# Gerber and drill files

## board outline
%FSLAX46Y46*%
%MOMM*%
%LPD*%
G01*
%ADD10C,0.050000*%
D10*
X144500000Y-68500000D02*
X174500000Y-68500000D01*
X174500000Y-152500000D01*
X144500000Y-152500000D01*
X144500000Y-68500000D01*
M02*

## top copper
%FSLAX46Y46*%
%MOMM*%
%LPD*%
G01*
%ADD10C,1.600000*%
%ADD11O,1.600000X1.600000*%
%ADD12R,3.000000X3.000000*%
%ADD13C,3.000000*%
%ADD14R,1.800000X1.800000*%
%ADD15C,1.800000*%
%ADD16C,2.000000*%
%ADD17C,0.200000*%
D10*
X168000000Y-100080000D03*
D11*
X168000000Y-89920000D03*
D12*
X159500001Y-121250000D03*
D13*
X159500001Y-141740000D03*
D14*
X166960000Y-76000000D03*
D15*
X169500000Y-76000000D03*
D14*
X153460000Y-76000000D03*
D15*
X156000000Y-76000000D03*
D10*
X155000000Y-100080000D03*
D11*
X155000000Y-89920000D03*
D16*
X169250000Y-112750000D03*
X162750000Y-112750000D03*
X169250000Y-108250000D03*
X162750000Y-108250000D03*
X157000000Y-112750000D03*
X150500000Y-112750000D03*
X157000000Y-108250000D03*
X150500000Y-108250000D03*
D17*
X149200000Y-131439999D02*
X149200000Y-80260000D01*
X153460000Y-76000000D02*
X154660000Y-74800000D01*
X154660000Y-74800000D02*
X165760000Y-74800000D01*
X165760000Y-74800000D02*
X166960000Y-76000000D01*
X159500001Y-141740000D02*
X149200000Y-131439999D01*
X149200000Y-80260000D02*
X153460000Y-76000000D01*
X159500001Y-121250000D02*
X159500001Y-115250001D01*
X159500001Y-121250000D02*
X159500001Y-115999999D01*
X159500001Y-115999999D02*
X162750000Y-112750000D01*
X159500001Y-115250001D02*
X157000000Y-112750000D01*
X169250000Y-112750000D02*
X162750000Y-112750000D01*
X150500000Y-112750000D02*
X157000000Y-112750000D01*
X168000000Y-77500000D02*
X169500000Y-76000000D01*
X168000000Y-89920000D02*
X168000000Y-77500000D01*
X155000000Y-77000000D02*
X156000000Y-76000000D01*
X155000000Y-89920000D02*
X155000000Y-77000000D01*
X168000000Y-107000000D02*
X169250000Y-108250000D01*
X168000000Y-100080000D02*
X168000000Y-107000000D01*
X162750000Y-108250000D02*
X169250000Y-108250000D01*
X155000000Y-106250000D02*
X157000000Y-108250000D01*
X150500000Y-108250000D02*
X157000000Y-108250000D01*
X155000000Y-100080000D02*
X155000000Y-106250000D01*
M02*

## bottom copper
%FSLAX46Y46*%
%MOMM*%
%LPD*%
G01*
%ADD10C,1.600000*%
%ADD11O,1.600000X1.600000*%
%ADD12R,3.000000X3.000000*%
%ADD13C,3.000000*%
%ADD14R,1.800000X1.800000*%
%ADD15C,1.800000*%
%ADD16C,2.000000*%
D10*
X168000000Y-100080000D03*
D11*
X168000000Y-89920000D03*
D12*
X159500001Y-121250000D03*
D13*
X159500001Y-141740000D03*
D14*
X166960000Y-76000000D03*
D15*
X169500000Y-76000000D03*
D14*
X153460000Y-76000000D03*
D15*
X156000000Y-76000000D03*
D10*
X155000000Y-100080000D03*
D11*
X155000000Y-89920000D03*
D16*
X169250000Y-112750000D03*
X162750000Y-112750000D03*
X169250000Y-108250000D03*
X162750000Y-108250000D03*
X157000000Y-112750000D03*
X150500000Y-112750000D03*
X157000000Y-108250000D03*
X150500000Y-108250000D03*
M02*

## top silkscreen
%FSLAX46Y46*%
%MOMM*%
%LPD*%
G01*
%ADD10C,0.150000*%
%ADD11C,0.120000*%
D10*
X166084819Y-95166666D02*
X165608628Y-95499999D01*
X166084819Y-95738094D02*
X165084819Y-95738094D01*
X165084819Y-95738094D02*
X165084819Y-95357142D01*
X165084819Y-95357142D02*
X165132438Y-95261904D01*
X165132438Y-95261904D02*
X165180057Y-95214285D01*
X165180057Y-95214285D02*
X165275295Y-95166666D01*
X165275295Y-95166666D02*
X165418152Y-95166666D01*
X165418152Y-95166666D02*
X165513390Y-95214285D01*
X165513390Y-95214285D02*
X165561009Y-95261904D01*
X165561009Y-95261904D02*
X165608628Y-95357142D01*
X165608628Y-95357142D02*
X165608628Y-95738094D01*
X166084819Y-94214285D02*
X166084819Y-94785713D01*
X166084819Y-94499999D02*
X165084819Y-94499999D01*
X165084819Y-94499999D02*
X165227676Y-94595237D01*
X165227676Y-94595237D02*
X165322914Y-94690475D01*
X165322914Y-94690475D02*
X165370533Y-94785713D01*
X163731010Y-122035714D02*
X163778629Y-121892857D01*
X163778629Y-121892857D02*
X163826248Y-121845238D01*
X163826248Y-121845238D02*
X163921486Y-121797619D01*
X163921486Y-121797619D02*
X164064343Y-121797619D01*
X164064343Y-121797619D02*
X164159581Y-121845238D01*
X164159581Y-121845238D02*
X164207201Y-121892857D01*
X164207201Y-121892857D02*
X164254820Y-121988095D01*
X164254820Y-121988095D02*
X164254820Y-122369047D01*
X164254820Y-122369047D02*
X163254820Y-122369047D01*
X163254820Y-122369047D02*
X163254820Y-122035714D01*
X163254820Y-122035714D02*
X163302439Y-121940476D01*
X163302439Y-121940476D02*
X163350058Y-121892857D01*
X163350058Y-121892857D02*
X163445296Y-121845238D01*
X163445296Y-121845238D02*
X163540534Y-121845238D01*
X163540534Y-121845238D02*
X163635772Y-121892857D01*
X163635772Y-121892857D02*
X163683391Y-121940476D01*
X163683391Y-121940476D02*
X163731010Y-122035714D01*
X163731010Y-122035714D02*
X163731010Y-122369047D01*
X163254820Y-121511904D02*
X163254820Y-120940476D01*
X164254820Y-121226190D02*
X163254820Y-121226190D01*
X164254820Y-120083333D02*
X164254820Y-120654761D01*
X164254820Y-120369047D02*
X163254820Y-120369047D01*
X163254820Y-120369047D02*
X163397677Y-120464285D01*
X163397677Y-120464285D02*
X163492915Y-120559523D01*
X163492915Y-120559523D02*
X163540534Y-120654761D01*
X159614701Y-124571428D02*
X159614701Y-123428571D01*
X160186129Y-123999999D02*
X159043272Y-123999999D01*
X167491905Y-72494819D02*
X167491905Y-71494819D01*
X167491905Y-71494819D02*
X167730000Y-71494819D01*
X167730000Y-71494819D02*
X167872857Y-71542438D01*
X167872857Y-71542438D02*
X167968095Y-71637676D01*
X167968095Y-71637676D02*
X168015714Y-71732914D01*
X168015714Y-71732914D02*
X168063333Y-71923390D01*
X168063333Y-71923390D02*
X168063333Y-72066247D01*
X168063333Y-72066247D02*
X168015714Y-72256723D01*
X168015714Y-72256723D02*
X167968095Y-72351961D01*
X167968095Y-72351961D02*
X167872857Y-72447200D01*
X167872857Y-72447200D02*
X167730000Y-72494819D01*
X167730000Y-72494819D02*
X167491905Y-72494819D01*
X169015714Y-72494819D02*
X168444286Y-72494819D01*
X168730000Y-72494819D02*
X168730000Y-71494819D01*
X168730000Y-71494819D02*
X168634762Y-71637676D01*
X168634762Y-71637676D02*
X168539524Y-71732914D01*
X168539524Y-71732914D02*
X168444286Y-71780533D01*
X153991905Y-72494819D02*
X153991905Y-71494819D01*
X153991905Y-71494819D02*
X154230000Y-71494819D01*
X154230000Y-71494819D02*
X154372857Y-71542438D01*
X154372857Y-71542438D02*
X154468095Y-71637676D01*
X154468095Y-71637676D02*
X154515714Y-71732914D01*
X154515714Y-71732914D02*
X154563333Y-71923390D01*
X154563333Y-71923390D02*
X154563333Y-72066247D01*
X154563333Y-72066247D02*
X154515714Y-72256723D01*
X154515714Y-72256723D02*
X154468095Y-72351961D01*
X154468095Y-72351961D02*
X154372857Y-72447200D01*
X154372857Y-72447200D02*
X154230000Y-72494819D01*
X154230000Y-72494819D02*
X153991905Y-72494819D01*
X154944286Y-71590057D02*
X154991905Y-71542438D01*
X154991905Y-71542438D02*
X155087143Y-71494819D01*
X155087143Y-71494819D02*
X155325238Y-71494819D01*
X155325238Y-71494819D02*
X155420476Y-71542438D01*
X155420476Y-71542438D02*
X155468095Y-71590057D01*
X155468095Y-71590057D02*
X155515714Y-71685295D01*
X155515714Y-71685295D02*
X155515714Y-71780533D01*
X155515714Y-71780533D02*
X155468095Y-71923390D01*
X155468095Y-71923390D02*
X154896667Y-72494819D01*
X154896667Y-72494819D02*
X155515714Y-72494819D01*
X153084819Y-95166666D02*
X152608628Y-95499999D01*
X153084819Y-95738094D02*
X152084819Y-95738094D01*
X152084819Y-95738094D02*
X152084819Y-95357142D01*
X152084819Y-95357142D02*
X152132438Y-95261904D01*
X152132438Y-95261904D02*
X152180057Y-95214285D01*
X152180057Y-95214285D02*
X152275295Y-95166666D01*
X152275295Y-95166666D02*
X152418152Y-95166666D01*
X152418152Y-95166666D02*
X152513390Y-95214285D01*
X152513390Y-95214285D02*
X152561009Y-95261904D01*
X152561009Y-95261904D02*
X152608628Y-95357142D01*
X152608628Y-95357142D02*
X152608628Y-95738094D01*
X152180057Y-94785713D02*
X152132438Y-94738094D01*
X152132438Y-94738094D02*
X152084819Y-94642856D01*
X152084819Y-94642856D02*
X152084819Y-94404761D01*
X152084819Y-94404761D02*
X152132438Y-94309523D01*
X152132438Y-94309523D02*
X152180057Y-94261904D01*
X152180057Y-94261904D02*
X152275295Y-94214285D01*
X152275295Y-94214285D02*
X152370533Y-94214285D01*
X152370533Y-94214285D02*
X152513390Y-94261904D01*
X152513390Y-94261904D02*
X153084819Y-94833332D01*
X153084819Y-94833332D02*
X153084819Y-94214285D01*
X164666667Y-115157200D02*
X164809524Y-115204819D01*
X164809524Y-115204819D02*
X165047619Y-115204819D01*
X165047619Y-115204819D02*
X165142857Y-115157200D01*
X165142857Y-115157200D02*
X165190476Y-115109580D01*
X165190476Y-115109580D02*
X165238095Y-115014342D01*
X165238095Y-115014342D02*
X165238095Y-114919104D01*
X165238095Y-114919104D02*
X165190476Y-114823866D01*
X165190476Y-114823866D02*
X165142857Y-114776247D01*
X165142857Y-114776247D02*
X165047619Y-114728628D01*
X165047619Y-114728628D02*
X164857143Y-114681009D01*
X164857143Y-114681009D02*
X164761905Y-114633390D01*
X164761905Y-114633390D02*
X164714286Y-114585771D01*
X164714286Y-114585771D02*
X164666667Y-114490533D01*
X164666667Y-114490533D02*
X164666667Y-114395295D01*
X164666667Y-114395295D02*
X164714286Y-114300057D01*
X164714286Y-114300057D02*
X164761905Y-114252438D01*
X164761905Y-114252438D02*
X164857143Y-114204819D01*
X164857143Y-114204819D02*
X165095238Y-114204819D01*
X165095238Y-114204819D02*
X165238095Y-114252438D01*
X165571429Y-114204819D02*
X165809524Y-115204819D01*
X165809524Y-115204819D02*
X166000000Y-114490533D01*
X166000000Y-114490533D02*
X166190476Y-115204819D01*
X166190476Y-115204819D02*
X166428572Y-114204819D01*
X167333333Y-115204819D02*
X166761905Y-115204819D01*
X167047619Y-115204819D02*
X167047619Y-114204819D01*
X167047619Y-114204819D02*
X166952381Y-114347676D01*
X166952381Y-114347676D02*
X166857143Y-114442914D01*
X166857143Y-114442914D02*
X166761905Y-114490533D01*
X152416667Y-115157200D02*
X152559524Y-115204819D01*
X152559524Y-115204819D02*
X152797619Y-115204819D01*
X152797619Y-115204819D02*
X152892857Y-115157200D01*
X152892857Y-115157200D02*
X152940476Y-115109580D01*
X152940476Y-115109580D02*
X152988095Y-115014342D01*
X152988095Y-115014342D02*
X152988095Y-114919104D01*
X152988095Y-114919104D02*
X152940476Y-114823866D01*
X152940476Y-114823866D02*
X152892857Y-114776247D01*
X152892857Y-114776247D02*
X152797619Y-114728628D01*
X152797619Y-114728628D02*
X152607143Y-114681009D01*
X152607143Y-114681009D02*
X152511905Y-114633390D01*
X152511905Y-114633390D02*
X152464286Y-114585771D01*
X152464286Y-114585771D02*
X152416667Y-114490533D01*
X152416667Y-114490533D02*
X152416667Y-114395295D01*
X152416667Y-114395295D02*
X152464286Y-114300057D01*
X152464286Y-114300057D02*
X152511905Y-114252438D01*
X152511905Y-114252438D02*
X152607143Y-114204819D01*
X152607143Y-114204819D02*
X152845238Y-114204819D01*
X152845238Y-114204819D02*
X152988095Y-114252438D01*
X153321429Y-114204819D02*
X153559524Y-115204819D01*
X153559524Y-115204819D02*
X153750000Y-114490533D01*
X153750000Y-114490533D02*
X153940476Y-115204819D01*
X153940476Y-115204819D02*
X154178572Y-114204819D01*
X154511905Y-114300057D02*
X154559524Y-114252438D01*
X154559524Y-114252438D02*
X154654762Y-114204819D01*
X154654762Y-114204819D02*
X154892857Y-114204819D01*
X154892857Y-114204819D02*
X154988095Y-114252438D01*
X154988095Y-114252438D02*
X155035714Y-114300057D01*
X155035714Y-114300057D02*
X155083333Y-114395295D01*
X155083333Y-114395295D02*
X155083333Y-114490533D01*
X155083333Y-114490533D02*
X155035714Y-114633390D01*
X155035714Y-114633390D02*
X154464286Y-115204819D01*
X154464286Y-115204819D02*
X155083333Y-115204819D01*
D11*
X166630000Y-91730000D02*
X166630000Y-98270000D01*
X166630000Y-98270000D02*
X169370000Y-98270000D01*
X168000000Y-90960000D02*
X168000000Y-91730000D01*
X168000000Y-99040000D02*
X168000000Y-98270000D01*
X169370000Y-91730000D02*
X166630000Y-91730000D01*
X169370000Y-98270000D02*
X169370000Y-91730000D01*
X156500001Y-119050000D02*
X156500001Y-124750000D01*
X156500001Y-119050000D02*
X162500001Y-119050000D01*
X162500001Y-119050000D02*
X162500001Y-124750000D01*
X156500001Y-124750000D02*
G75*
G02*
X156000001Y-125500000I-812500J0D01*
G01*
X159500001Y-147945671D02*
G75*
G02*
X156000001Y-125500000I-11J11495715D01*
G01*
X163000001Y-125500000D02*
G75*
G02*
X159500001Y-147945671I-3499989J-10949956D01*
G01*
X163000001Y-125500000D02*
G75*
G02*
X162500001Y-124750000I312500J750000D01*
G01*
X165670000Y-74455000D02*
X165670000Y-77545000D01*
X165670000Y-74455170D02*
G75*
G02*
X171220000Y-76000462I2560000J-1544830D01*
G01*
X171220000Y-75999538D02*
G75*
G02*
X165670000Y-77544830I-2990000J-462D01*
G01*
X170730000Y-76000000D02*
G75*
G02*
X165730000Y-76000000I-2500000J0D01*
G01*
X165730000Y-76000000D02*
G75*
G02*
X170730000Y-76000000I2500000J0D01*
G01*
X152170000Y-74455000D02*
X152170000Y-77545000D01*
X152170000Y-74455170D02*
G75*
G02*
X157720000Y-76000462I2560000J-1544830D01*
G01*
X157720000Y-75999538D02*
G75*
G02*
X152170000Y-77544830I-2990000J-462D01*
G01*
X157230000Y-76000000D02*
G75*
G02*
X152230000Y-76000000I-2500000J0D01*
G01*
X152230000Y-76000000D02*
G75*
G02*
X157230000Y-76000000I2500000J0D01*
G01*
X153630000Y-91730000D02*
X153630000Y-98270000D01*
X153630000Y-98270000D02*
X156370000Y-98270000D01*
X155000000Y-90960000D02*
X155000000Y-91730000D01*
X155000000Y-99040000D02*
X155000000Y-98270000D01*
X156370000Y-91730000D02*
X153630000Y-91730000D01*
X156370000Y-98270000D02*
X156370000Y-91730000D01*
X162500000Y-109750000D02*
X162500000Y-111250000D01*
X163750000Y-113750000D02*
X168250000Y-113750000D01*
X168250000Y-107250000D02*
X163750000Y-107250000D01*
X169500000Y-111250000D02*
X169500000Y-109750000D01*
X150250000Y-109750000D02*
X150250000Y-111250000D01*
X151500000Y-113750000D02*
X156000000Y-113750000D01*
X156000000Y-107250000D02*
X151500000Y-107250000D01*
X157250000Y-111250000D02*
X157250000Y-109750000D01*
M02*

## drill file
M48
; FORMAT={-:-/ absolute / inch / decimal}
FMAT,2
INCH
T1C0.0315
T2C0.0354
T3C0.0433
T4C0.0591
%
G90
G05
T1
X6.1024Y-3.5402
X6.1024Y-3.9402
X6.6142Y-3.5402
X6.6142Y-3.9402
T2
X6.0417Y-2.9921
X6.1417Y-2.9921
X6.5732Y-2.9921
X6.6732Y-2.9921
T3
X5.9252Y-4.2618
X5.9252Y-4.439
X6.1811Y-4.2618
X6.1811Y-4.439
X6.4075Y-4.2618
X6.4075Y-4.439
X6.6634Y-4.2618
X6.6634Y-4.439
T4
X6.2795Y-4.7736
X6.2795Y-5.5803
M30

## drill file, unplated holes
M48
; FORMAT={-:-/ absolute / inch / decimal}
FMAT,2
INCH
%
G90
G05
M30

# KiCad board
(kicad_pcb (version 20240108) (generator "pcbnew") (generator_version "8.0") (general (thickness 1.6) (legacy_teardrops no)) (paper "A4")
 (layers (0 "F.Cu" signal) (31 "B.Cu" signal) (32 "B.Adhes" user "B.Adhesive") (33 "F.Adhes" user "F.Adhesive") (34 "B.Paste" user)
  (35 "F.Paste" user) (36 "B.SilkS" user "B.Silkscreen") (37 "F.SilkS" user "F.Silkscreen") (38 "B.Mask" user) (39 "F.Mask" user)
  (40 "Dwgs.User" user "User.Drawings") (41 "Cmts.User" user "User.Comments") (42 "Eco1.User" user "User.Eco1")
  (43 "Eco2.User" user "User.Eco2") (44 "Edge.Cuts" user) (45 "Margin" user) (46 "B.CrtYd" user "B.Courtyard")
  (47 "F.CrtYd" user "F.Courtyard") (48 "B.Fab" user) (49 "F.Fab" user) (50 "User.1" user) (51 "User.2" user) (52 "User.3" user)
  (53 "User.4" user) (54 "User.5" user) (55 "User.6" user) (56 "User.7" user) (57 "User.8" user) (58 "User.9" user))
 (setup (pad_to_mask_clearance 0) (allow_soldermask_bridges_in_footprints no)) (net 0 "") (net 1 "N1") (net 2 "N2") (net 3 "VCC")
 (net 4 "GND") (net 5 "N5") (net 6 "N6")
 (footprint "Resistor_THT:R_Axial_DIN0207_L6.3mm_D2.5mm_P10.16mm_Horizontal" (layer "F.Cu") (at 168 100.08 90)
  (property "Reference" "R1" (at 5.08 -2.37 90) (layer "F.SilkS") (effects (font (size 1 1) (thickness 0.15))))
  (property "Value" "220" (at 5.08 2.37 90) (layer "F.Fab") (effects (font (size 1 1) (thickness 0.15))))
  (fp_line (start 8.35 -1.37) (end 1.81 -1.37) (stroke (width 0.12) (type solid)) (layer "F.SilkS"))
  (fp_line (start 1.81 -1.37) (end 1.81 1.37) (stroke (width 0.12) (type solid)) (layer "F.SilkS"))
  (fp_line (start 9.12 0) (end 8.35 0) (stroke (width 0.12) (type solid)) (layer "F.SilkS"))
  (fp_line (start 1.04 0) (end 1.81 0) (stroke (width 0.12) (type solid)) (layer "F.SilkS"))
  (fp_line (start 8.35 1.37) (end 8.35 -1.37) (stroke (width 0.12) (type solid)) (layer "F.SilkS"))
  (fp_line (start 1.81 1.37) (end 8.35 1.37) (stroke (width 0.12) (type solid)) (layer "F.SilkS"))
  (pad "1" thru_hole circle (at 0 0 90) (size 1.6 1.6) (drill 0.8) (layers "*.Cu" "*.Mask") (remove_unused_layers no) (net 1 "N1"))
  (pad "2" thru_hole oval (at 10.16 0 90) (size 1.6 1.6) (drill 0.8) (layers "*.Cu" "*.Mask") (remove_unused_layers no) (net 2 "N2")))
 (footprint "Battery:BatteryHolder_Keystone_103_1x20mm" (layer "F.Cu") (at 159.500001 121.25 -90)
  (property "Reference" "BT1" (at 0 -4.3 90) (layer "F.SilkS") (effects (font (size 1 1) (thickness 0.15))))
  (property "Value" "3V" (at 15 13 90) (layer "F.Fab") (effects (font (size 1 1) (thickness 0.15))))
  (fp_line (start -2.2 3) (end 3.5 3) (stroke (width 0.12) (type solid)) (layer "F.SilkS"))
  (fp_line (start -2.2 3) (end -2.2 -3) (stroke (width 0.12) (type solid)) (layer "F.SilkS"))
  (fp_line (start -2.2 -3) (end 3.5 -3) (stroke (width 0.12) (type solid)) (layer "F.SilkS"))
  (fp_arc (start 3.5 3) (mid 3.950694 3.136459) (end 4.25 3.5) (stroke (width 0.12) (type solid)) (layer "F.SilkS"))
  (fp_arc (start 26.695671 0) (mid 16.971103 11.358466) (end 4.25 3.5) (stroke (width 0.12) (type solid)) (layer "F.SilkS"))
  (fp_arc (start 4.25 -3.5) (mid 16.971103 -11.358466) (end 26.695671 0) (stroke (width 0.12) (type solid)) (layer "F.SilkS"))
  (fp_arc (start 4.25 -3.5) (mid 3.950694 -3.136459) (end 3.5 -3) (stroke (width 0.12) (type solid)) (layer "F.SilkS"))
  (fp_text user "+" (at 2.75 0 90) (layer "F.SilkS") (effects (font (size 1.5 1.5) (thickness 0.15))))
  (pad "1" thru_hole rect (at 0 0 270) (size 3 3) (drill 1.5) (layers "*.Cu" "*.Mask") (remove_unused_layers no) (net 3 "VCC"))
  (pad "2" thru_hole circle (at 20.49 0 270) (size 3 3) (drill 1.5) (layers "*.Cu" "*.Mask") (remove_unused_layers no) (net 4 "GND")))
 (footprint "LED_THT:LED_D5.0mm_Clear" (layer "F.Cu") (at 166.96 76)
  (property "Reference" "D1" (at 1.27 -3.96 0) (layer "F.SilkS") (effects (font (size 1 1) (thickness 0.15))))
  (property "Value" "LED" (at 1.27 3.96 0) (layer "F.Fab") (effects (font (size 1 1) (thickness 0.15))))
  (fp_line (start -1.29 -1.545) (end -1.29 1.545) (stroke (width 0.12) (type solid)) (layer "F.SilkS"))
  (fp_arc (start -1.29 -1.54483) (mid 2.072002 -2.880433) (end 4.26 0.000462) (stroke (width 0.12) (type solid)) (layer "F.SilkS"))
  (fp_arc (start 4.26 -0.000462) (mid 2.072002 2.880433) (end -1.29 1.54483) (stroke (width 0.12) (type solid)) (layer "F.SilkS"))
  (fp_circle (center 1.27 0) (end 3.77 0) (stroke (width 0.12) (type solid)) (fill none) (layer "F.SilkS"))
  (pad "1" thru_hole rect (at 0 0) (size 1.8 1.8) (drill 0.9) (layers "*.Cu" "*.Mask") (remove_unused_layers no) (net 4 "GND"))
  (pad "2" thru_hole circle (at 2.54 0) (size 1.8 1.8) (drill 0.9) (layers "*.Cu" "*.Mask") (remove_unused_layers no) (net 2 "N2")))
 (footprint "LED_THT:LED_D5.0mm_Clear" (layer "F.Cu") (at 153.46 76)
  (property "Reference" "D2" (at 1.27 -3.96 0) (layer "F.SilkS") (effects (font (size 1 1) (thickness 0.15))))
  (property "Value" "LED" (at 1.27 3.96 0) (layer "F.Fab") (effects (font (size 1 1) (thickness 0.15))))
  (fp_line (start -1.29 -1.545) (end -1.29 1.545) (stroke (width 0.12) (type solid)) (layer "F.SilkS"))
  (fp_arc (start -1.29 -1.54483) (mid 2.072002 -2.880433) (end 4.26 0.000462) (stroke (width 0.12) (type solid)) (layer "F.SilkS"))
  (fp_arc (start 4.26 -0.000462) (mid 2.072002 2.880433) (end -1.29 1.54483) (stroke (width 0.12) (type solid)) (layer "F.SilkS"))
  (fp_circle (center 1.27 0) (end 3.77 0) (stroke (width 0.12) (type solid)) (fill none) (layer "F.SilkS"))
  (pad "1" thru_hole rect (at 0 0) (size 1.8 1.8) (drill 0.9) (layers "*.Cu" "*.Mask") (remove_unused_layers no) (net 4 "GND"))
  (pad "2" thru_hole circle (at 2.54 0) (size 1.8 1.8) (drill 0.9) (layers "*.Cu" "*.Mask") (remove_unused_layers no) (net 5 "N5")))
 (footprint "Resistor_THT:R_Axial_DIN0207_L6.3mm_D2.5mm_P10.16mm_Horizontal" (layer "F.Cu") (at 155 100.08 90)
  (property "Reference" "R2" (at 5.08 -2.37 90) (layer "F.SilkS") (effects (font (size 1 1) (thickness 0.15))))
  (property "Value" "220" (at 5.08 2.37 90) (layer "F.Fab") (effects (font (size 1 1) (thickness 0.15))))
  (fp_line (start 8.35 -1.37) (end 1.81 -1.37) (stroke (width 0.12) (type solid)) (layer "F.SilkS"))
  (fp_line (start 1.81 -1.37) (end 1.81 1.37) (stroke (width 0.12) (type solid)) (layer "F.SilkS"))
  (fp_line (start 9.12 0) (end 8.35 0) (stroke (width 0.12) (type solid)) (layer "F.SilkS"))
  (fp_line (start 1.04 0) (end 1.81 0) (stroke (width 0.12) (type solid)) (layer "F.SilkS"))
  (fp_line (start 8.35 1.37) (end 8.35 -1.37) (stroke (width 0.12) (type solid)) (layer "F.SilkS"))
  (fp_line (start 1.81 1.37) (end 8.35 1.37) (stroke (width 0.12) (type solid)) (layer "F.SilkS"))
  (pad "1" thru_hole circle (at 0 0 90) (size 1.6 1.6) (drill 0.8) (layers "*.Cu" "*.Mask") (remove_unused_layers no) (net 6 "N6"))
  (pad "2" thru_hole oval (at 10.16 0 90) (size 1.6 1.6) (drill 0.8) (layers "*.Cu" "*.Mask") (remove_unused_layers no) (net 5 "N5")))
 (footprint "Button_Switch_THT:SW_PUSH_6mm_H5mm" (layer "F.Cu") (at 169.25 112.75 180)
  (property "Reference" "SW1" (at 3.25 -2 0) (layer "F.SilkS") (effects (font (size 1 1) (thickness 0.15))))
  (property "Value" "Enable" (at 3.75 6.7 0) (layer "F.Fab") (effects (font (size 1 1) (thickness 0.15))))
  (fp_line (start 6.75 3) (end 6.75 1.5) (stroke (width 0.12) (type solid)) (layer "F.SilkS"))
  (fp_line (start 5.5 -1) (end 1 -1) (stroke (width 0.12) (type solid)) (layer "F.SilkS"))
  (fp_line (start 1 5.5) (end 5.5 5.5) (stroke (width 0.12) (type solid)) (layer "F.SilkS"))
  (fp_line (start -0.25 1.5) (end -0.25 3) (stroke (width 0.12) (type solid)) (layer "F.SilkS"))
  (pad "1" thru_hole circle (at 0 0 270) (size 2 2) (drill 1.1) (layers "*.Cu" "*.Mask") (remove_unused_layers no) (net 3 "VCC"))
  (pad "1" thru_hole circle (at 6.5 0 270) (size 2 2) (drill 1.1) (layers "*.Cu" "*.Mask") (remove_unused_layers no) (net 3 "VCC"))
  (pad "2" thru_hole circle (at 0 4.5 270) (size 2 2) (drill 1.1) (layers "*.Cu" "*.Mask") (remove_unused_layers no) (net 1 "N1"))
  (pad "2" thru_hole circle (at 6.5 4.5 270) (size 2 2) (drill 1.1) (layers "*.Cu" "*.Mask") (remove_unused_layers no) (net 1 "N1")))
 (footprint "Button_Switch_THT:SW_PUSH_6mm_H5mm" (layer "F.Cu") (at 157 112.75 180)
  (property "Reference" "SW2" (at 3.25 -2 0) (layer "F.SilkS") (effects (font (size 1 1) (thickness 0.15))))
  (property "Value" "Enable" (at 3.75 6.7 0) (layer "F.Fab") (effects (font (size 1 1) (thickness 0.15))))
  (fp_line (start 6.75 3) (end 6.75 1.5) (stroke (width 0.12) (type solid)) (layer "F.SilkS"))
  (fp_line (start 5.5 -1) (end 1 -1) (stroke (width 0.12) (type solid)) (layer "F.SilkS"))
  (fp_line (start 1 5.5) (end 5.5 5.5) (stroke (width 0.12) (type solid)) (layer "F.SilkS"))
  (fp_line (start -0.25 1.5) (end -0.25 3) (stroke (width 0.12) (type solid)) (layer "F.SilkS"))
  (pad "1" thru_hole circle (at 0 0 270) (size 2 2) (drill 1.1) (layers "*.Cu" "*.Mask") (remove_unused_layers no) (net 3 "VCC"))
  (pad "1" thru_hole circle (at 6.5 0 270) (size 2 2) (drill 1.1) (layers "*.Cu" "*.Mask") (remove_unused_layers no) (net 3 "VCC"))
  (pad "2" thru_hole circle (at 0 4.5 270) (size 2 2) (drill 1.1) (layers "*.Cu" "*.Mask") (remove_unused_layers no) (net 6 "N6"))
  (pad "2" thru_hole circle (at 6.5 4.5 270) (size 2 2) (drill 1.1) (layers "*.Cu" "*.Mask") (remove_unused_layers no) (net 6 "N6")))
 (gr_rect (start 144.5 68.5) (end 174.5 152.5) (stroke (width 0.05) (type default)) (fill none) (layer "Edge.Cuts"))
 (segment (start 149.2 131.439999) (end 149.2 80.26) (width 0.2) (layer "F.Cu") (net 4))
 (segment (start 153.46 76) (end 154.66 74.8) (width 0.2) (layer "F.Cu") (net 4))
 (segment (start 154.66 74.8) (end 165.76 74.8) (width 0.2) (layer "F.Cu") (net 4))
 (segment (start 165.76 74.8) (end 166.96 76) (width 0.2) (layer "F.Cu") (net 4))
 (segment (start 159.500001 141.74) (end 149.2 131.439999) (width 0.2) (layer "F.Cu") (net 4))
 (segment (start 149.2 80.26) (end 153.46 76) (width 0.2) (layer "F.Cu") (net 4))
 (segment (start 159.500001 121.25) (end 159.500001 115.250001) (width 0.2) (layer "F.Cu") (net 3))
 (segment (start 159.500001 121.25) (end 159.500001 115.999999) (width 0.2) (layer "F.Cu") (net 3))
 (segment (start 159.500001 115.999999) (end 162.75 112.75) (width 0.2) (layer "F.Cu") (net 3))
 (segment (start 159.500001 115.250001) (end 157 112.75) (width 0.2) (layer "F.Cu") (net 3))
 (segment (start 169.25 112.75) (end 162.75 112.75) (width 0.2) (layer "F.Cu") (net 3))
 (segment (start 150.5 112.75) (end 157 112.75) (width 0.2) (layer "F.Cu") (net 3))
 (segment (start 168 77.5) (end 169.5 76) (width 0.2) (layer "F.Cu") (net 2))
 (segment (start 168 89.92) (end 168 77.5) (width 0.2) (layer "F.Cu") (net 2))
 (segment (start 155 77) (end 156 76) (width 0.2) (layer "F.Cu") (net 5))
 (segment (start 155 89.92) (end 155 77) (width 0.2) (layer "F.Cu") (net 5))
 (segment (start 168 107) (end 169.25 108.25) (width 0.2) (layer "F.Cu") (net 1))
 (segment (start 168 100.08) (end 168 107) (width 0.2) (layer "F.Cu") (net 1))
 (segment (start 162.75 108.25) (end 169.25 108.25) (width 0.2) (layer "F.Cu") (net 1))
 (segment (start 155 106.25) (end 157 108.25) (width 0.2) (layer "F.Cu") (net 6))
 (segment (start 150.5 108.25) (end 157 108.25) (width 0.2) (layer "F.Cu") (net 6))
 (segment (start 155 100.08) (end 155 106.25) (width 0.2) (layer "F.Cu") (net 6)))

